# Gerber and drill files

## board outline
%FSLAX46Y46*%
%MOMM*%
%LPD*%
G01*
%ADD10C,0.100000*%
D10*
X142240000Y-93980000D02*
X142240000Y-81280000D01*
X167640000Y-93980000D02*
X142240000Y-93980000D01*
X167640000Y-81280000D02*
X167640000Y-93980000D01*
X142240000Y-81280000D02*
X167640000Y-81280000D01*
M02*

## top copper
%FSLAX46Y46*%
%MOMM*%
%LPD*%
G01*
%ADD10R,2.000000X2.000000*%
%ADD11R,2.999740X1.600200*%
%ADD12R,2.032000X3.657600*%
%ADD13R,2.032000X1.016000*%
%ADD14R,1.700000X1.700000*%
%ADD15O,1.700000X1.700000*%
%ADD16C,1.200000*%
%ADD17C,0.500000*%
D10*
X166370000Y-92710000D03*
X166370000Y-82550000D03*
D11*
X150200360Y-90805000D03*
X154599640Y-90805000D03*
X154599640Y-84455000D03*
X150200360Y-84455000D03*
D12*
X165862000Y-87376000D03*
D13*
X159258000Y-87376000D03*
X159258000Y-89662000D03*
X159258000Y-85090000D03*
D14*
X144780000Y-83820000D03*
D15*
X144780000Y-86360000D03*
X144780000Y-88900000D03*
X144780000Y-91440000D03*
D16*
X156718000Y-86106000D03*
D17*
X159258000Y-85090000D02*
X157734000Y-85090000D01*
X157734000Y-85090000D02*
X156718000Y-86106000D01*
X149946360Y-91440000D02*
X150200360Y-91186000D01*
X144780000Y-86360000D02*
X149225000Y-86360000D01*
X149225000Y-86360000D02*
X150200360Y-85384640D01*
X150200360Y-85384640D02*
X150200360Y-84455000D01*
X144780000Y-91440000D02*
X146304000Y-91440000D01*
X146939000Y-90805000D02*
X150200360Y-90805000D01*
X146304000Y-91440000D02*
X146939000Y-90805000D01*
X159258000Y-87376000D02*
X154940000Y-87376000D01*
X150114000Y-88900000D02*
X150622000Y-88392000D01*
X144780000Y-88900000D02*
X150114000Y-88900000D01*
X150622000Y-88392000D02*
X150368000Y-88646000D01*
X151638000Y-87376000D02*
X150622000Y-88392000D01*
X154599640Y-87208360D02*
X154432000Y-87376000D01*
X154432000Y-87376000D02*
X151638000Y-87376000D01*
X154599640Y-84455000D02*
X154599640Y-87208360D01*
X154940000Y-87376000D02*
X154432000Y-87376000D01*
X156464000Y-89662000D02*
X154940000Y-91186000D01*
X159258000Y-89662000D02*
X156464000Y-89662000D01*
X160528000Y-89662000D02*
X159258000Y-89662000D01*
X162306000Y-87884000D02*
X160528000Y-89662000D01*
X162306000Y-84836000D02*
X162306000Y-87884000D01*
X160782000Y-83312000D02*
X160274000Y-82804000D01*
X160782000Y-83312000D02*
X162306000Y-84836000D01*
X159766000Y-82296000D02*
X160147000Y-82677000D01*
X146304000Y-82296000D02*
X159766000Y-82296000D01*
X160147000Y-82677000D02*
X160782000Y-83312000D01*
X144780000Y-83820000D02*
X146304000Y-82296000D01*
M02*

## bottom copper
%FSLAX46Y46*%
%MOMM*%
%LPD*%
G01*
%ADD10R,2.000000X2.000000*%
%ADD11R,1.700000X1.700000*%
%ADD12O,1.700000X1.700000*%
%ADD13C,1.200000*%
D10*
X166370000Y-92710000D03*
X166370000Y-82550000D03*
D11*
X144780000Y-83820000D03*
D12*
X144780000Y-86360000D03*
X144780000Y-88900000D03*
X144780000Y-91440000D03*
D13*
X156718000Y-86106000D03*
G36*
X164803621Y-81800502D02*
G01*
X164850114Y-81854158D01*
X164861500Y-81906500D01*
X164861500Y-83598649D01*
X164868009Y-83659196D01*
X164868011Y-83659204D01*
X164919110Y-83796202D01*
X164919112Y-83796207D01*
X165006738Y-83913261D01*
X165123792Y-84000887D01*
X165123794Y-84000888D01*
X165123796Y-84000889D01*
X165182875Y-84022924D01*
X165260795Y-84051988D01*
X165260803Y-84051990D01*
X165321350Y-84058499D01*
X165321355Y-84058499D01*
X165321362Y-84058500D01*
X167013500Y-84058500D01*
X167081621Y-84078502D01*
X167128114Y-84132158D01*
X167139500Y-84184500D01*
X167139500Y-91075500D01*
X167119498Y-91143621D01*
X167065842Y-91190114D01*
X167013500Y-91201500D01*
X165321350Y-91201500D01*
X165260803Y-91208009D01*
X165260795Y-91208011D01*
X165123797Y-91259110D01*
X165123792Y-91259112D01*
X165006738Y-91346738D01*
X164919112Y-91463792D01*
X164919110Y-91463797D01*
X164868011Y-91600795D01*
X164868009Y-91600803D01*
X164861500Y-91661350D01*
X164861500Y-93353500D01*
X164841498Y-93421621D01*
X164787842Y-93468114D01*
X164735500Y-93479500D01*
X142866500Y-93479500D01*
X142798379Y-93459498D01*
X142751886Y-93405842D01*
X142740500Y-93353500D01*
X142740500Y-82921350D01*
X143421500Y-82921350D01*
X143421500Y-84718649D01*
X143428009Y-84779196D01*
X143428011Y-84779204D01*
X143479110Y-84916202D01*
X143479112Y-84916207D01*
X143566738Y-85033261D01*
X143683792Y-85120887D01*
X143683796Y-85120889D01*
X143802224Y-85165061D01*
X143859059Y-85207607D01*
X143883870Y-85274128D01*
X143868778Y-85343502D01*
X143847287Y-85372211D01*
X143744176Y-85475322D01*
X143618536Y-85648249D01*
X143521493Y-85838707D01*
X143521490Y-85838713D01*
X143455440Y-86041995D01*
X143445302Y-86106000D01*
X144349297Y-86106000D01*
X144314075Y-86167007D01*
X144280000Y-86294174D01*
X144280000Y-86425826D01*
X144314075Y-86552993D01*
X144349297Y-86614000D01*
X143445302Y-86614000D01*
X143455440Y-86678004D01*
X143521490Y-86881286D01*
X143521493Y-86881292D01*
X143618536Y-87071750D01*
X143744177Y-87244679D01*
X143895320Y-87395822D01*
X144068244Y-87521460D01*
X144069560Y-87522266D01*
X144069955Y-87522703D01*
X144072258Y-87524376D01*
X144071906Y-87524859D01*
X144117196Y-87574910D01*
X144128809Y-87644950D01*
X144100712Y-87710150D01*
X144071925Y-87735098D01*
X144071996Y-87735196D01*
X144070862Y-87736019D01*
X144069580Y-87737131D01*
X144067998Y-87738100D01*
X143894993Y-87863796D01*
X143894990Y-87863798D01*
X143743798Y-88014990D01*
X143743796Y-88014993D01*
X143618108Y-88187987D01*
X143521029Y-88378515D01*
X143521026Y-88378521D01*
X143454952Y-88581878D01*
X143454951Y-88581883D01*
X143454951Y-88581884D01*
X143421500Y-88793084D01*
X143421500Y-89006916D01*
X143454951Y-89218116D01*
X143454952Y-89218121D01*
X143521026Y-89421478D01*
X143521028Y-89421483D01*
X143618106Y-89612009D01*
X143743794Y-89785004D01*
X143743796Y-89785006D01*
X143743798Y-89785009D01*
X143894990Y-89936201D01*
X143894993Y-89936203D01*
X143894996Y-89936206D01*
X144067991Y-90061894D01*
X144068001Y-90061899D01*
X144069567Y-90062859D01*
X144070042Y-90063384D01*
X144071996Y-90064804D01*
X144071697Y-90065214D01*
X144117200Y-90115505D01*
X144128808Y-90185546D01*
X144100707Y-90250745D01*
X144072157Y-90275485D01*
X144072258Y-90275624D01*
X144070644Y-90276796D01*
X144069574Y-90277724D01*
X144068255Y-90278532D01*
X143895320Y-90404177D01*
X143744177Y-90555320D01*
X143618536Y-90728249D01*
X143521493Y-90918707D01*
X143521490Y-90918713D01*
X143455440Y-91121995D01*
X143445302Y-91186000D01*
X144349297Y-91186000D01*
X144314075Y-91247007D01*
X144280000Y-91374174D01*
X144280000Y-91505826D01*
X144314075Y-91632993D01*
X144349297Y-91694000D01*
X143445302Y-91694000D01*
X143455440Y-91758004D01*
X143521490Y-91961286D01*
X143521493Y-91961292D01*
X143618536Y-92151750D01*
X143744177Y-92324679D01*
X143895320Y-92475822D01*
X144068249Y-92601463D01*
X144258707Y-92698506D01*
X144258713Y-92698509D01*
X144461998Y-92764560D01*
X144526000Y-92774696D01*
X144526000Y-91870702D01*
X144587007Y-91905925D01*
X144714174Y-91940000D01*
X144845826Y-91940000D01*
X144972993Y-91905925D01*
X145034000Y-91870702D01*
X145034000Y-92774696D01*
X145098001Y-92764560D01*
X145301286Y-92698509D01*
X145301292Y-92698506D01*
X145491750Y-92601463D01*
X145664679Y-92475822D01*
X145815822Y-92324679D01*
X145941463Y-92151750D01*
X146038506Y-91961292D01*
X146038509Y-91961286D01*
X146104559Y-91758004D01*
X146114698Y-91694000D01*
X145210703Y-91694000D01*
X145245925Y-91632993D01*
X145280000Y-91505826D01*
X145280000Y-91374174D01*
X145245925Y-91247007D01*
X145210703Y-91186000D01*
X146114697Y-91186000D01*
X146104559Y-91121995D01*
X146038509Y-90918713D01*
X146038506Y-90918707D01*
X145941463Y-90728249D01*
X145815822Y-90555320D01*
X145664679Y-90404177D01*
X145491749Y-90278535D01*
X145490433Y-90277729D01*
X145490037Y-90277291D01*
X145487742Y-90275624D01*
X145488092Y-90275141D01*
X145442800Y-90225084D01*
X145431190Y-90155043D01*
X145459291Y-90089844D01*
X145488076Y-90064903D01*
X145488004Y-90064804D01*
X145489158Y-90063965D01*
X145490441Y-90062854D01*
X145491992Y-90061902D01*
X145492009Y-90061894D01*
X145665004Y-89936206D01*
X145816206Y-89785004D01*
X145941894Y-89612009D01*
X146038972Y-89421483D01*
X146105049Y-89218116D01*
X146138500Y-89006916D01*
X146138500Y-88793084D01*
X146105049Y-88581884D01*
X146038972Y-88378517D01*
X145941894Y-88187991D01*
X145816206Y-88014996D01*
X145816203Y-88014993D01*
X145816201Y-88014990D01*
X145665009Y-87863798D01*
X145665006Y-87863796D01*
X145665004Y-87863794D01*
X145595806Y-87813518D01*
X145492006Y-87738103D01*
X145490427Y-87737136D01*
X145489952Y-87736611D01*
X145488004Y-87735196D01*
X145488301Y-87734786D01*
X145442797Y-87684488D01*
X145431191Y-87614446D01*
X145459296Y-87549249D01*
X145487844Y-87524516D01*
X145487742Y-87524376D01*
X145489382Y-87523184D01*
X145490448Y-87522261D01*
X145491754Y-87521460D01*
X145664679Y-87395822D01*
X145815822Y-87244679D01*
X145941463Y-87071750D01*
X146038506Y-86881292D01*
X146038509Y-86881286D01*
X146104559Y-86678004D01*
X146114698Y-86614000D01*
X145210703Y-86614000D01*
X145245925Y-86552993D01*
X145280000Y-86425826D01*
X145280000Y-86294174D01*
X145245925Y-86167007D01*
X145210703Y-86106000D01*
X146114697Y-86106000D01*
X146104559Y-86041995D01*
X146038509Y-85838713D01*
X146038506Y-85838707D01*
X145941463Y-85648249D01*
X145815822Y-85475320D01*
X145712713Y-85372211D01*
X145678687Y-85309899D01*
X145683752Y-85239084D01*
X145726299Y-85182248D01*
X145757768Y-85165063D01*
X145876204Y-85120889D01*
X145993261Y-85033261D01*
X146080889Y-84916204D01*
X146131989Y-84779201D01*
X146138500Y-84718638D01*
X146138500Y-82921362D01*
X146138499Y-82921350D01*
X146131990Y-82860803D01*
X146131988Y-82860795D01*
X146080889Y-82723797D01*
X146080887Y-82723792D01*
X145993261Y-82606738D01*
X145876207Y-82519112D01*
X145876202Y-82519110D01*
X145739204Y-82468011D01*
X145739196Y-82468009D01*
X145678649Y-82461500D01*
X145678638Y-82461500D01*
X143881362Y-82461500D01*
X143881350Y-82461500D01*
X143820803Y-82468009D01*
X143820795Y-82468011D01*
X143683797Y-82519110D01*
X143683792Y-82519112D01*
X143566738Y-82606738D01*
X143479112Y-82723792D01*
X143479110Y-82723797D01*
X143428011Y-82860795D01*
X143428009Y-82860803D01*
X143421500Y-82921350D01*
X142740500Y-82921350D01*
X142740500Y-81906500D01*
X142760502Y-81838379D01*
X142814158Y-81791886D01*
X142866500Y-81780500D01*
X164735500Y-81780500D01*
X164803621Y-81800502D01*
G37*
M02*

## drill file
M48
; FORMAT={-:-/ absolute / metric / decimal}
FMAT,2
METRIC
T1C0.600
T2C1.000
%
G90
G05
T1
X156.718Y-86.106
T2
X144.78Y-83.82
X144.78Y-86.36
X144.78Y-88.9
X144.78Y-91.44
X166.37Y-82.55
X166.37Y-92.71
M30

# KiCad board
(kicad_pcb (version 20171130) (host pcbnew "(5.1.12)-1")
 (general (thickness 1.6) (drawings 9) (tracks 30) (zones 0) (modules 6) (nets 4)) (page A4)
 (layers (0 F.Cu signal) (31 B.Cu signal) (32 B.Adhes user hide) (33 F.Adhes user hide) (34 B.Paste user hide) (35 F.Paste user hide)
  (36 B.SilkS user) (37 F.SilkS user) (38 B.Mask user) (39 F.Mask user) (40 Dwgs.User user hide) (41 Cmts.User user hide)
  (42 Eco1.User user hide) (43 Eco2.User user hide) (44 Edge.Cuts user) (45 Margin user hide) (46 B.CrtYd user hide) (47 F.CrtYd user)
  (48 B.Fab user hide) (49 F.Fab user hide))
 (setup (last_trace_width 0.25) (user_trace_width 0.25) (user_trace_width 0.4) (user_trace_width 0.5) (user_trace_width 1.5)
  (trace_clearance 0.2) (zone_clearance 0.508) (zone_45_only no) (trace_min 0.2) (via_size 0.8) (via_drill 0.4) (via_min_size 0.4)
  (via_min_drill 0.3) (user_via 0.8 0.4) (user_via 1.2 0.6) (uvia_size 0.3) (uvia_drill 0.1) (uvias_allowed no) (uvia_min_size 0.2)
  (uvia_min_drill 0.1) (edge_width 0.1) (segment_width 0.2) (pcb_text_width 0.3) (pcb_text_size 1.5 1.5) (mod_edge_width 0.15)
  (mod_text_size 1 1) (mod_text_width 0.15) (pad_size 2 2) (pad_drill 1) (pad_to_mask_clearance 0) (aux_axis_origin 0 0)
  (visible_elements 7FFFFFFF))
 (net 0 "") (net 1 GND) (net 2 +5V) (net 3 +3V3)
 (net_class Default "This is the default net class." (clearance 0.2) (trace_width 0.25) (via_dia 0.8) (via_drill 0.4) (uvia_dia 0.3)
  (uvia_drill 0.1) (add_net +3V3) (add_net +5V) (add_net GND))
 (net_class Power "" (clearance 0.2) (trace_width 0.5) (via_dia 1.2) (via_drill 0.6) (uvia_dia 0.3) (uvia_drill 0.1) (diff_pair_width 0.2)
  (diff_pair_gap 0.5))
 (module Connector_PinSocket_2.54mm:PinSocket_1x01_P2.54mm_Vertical (layer F.Cu) (at 166.37 92.71)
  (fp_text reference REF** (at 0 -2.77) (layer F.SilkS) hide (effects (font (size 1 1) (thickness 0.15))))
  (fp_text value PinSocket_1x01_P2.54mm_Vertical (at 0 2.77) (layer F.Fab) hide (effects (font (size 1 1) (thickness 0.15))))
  (pad 1 thru_hole rect (at 0 0) (size 2 2) (drill 1) (layers *.Cu *.Mask)))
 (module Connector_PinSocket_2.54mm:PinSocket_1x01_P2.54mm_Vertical (layer F.Cu) (at 166.37 82.55)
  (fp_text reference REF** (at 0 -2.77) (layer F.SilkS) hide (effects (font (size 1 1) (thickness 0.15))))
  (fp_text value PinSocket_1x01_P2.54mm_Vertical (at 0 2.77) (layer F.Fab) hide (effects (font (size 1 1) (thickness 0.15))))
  (pad 1 thru_hole rect (at 0 0) (size 2 2) (drill 1) (layers *.Cu *.Mask)))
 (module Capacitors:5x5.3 (layer F.Cu) (at 152.4 90.805)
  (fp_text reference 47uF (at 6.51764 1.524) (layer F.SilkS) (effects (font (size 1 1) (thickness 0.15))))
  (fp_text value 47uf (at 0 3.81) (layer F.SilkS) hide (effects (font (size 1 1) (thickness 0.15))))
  (pad 2 smd rect (at -2.19964 0) (size 2.99974 1.6002) (layers F.Cu F.Paste F.Mask) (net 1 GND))
  (pad 1 smd rect (at 2.19964 0) (size 2.99974 1.6002) (layers F.Cu F.Paste F.Mask) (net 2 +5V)))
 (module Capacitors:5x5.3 (layer F.Cu) (at 152.4 84.455)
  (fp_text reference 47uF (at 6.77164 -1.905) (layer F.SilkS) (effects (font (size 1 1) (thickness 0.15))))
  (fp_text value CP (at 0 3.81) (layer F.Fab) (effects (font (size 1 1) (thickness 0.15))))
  (pad 1 smd rect (at 2.19964 0) (size 2.99974 1.6002) (layers F.Cu F.Paste F.Mask) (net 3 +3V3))
  (pad 2 smd rect (at -2.19964 0) (size 2.99974 1.6002) (layers F.Cu F.Paste F.Mask) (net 1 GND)))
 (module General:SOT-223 (layer F.Cu) (at 162.56 87.376 270)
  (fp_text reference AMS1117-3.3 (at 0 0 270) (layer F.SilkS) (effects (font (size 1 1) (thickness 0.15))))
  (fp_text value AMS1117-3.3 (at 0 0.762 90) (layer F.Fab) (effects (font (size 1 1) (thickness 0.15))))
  (pad 4 smd rect (at 0 -3.302 270) (size 3.6576 2.032) (layers F.Cu F.Paste F.Mask))
  (pad 2 smd rect (at 0 3.302 270) (size 1.016 2.032) (layers F.Cu F.Paste F.Mask) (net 3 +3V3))
  (pad 3 smd rect (at 2.286 3.302 270) (size 1.016 2.032) (layers F.Cu F.Paste F.Mask) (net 2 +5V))
  (pad 1 smd rect (at -2.286 3.302 270) (size 1.016 2.032) (layers F.Cu F.Paste F.Mask) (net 1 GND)))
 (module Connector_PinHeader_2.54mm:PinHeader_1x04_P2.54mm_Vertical (layer F.Cu) (at 144.78 83.82)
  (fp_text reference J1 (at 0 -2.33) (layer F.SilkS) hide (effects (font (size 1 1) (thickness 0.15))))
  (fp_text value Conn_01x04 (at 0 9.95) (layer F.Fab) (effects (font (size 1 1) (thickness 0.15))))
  (pad 1 thru_hole rect (at 0 0) (size 1.7 1.7) (drill 1) (layers *.Cu *.Mask) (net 2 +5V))
  (pad 2 thru_hole oval (at 0 2.54) (size 1.7 1.7) (drill 1) (layers *.Cu *.Mask) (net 1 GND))
  (pad 3 thru_hole oval (at 0 5.08) (size 1.7 1.7) (drill 1) (layers *.Cu *.Mask) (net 3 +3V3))
  (pad 4 thru_hole oval (at 0 7.62) (size 1.7 1.7) (drill 1) (layers *.Cu *.Mask) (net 1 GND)))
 (gr_line (start 142.24 93.98) (end 142.24 81.28) (layer Edge.Cuts) (width 0.1))
 (gr_line (start 167.64 93.98) (end 142.24 93.98) (layer Edge.Cuts) (width 0.1))
 (gr_line (start 167.64 81.28) (end 167.64 93.98) (layer Edge.Cuts) (width 0.1))
 (gr_line (start 142.24 81.28) (end 167.64 81.28) (layer Edge.Cuts) (width 0.1))
 (segment (start 159.258 85.09) (end 157.734 85.09) (width 0.5) (layer F.Cu) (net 1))
 (segment (start 157.734 85.09) (end 156.718 86.106) (width 0.5) (layer F.Cu) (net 1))
 (via (at 156.718 86.106) (size 1.2) (drill 0.6) (layers F.Cu B.Cu) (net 1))
 (segment (start 149.94636 91.44) (end 150.20036 91.186) (width 0.5) (layer F.Cu) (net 1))
 (segment (start 144.78 86.36) (end 149.225 86.36) (width 0.5) (layer F.Cu) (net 1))
 (segment (start 149.225 86.36) (end 150.20036 85.38464) (width 0.5) (layer F.Cu) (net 1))
 (segment (start 150.20036 85.38464) (end 150.20036 84.455) (width 0.5) (layer F.Cu) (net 1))
 (segment (start 144.78 91.44) (end 146.304 91.44) (width 0.5) (layer F.Cu) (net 1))
 (segment (start 146.939 90.805) (end 150.20036 90.805) (width 0.5) (layer F.Cu) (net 1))
 (segment (start 146.304 91.44) (end 146.939 90.805) (width 0.5) (layer F.Cu) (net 1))
 (segment (start 159.258 87.376) (end 154.94 87.376) (width 0.5) (layer F.Cu) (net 3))
 (segment (start 150.114 88.9) (end 150.622 88.392) (width 0.5) (layer F.Cu) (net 3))
 (segment (start 144.78 88.9) (end 150.114 88.9) (width 0.5) (layer F.Cu) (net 3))
 (segment (start 150.622 88.392) (end 150.368 88.646) (width 0.5) (layer F.Cu) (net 3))
 (segment (start 151.638 87.376) (end 150.622 88.392) (width 0.5) (layer F.Cu) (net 3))
 (segment (start 154.59964 87.20836) (end 154.432 87.376) (width 0.5) (layer F.Cu) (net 3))
 (segment (start 154.432 87.376) (end 151.638 87.376) (width 0.5) (layer F.Cu) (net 3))
 (segment (start 154.59964 84.455) (end 154.59964 87.20836) (width 0.5) (layer F.Cu) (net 3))
 (segment (start 154.94 87.376) (end 154.432 87.376) (width 0.5) (layer F.Cu) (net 3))
 (segment (start 156.464 89.662) (end 154.94 91.186) (width 0.5) (layer F.Cu) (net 2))
 (segment (start 159.258 89.662) (end 156.464 89.662) (width 0.5) (layer F.Cu) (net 2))
 (segment (start 160.528 89.662) (end 159.258 89.662) (width 0.5) (layer F.Cu) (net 2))
 (segment (start 162.306 87.884) (end 160.528 89.662) (width 0.5) (layer F.Cu) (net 2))
 (segment (start 162.306 84.836) (end 162.306 87.884) (width 0.5) (layer F.Cu) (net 2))
 (segment (start 160.782 83.312) (end 160.274 82.804) (width 0.5) (layer F.Cu) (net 2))
 (segment (start 160.782 83.312) (end 162.306 84.836) (width 0.5) (layer F.Cu) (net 2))
 (segment (start 159.766 82.296) (end 160.147 82.677) (width 0.5) (layer F.Cu) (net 2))
 (segment (start 146.304 82.296) (end 159.766 82.296) (width 0.5) (layer F.Cu) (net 2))
 (segment (start 160.147 82.677) (end 160.782 83.312) (width 0.5) (layer F.Cu) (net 2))
 (segment (start 144.78 83.82) (end 146.304 82.296) (width 0.5) (layer F.Cu) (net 2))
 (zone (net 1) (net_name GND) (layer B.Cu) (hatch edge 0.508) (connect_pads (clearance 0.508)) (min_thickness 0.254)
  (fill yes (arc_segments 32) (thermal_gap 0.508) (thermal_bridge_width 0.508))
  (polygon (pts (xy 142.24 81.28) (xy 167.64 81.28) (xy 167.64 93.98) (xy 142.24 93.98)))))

